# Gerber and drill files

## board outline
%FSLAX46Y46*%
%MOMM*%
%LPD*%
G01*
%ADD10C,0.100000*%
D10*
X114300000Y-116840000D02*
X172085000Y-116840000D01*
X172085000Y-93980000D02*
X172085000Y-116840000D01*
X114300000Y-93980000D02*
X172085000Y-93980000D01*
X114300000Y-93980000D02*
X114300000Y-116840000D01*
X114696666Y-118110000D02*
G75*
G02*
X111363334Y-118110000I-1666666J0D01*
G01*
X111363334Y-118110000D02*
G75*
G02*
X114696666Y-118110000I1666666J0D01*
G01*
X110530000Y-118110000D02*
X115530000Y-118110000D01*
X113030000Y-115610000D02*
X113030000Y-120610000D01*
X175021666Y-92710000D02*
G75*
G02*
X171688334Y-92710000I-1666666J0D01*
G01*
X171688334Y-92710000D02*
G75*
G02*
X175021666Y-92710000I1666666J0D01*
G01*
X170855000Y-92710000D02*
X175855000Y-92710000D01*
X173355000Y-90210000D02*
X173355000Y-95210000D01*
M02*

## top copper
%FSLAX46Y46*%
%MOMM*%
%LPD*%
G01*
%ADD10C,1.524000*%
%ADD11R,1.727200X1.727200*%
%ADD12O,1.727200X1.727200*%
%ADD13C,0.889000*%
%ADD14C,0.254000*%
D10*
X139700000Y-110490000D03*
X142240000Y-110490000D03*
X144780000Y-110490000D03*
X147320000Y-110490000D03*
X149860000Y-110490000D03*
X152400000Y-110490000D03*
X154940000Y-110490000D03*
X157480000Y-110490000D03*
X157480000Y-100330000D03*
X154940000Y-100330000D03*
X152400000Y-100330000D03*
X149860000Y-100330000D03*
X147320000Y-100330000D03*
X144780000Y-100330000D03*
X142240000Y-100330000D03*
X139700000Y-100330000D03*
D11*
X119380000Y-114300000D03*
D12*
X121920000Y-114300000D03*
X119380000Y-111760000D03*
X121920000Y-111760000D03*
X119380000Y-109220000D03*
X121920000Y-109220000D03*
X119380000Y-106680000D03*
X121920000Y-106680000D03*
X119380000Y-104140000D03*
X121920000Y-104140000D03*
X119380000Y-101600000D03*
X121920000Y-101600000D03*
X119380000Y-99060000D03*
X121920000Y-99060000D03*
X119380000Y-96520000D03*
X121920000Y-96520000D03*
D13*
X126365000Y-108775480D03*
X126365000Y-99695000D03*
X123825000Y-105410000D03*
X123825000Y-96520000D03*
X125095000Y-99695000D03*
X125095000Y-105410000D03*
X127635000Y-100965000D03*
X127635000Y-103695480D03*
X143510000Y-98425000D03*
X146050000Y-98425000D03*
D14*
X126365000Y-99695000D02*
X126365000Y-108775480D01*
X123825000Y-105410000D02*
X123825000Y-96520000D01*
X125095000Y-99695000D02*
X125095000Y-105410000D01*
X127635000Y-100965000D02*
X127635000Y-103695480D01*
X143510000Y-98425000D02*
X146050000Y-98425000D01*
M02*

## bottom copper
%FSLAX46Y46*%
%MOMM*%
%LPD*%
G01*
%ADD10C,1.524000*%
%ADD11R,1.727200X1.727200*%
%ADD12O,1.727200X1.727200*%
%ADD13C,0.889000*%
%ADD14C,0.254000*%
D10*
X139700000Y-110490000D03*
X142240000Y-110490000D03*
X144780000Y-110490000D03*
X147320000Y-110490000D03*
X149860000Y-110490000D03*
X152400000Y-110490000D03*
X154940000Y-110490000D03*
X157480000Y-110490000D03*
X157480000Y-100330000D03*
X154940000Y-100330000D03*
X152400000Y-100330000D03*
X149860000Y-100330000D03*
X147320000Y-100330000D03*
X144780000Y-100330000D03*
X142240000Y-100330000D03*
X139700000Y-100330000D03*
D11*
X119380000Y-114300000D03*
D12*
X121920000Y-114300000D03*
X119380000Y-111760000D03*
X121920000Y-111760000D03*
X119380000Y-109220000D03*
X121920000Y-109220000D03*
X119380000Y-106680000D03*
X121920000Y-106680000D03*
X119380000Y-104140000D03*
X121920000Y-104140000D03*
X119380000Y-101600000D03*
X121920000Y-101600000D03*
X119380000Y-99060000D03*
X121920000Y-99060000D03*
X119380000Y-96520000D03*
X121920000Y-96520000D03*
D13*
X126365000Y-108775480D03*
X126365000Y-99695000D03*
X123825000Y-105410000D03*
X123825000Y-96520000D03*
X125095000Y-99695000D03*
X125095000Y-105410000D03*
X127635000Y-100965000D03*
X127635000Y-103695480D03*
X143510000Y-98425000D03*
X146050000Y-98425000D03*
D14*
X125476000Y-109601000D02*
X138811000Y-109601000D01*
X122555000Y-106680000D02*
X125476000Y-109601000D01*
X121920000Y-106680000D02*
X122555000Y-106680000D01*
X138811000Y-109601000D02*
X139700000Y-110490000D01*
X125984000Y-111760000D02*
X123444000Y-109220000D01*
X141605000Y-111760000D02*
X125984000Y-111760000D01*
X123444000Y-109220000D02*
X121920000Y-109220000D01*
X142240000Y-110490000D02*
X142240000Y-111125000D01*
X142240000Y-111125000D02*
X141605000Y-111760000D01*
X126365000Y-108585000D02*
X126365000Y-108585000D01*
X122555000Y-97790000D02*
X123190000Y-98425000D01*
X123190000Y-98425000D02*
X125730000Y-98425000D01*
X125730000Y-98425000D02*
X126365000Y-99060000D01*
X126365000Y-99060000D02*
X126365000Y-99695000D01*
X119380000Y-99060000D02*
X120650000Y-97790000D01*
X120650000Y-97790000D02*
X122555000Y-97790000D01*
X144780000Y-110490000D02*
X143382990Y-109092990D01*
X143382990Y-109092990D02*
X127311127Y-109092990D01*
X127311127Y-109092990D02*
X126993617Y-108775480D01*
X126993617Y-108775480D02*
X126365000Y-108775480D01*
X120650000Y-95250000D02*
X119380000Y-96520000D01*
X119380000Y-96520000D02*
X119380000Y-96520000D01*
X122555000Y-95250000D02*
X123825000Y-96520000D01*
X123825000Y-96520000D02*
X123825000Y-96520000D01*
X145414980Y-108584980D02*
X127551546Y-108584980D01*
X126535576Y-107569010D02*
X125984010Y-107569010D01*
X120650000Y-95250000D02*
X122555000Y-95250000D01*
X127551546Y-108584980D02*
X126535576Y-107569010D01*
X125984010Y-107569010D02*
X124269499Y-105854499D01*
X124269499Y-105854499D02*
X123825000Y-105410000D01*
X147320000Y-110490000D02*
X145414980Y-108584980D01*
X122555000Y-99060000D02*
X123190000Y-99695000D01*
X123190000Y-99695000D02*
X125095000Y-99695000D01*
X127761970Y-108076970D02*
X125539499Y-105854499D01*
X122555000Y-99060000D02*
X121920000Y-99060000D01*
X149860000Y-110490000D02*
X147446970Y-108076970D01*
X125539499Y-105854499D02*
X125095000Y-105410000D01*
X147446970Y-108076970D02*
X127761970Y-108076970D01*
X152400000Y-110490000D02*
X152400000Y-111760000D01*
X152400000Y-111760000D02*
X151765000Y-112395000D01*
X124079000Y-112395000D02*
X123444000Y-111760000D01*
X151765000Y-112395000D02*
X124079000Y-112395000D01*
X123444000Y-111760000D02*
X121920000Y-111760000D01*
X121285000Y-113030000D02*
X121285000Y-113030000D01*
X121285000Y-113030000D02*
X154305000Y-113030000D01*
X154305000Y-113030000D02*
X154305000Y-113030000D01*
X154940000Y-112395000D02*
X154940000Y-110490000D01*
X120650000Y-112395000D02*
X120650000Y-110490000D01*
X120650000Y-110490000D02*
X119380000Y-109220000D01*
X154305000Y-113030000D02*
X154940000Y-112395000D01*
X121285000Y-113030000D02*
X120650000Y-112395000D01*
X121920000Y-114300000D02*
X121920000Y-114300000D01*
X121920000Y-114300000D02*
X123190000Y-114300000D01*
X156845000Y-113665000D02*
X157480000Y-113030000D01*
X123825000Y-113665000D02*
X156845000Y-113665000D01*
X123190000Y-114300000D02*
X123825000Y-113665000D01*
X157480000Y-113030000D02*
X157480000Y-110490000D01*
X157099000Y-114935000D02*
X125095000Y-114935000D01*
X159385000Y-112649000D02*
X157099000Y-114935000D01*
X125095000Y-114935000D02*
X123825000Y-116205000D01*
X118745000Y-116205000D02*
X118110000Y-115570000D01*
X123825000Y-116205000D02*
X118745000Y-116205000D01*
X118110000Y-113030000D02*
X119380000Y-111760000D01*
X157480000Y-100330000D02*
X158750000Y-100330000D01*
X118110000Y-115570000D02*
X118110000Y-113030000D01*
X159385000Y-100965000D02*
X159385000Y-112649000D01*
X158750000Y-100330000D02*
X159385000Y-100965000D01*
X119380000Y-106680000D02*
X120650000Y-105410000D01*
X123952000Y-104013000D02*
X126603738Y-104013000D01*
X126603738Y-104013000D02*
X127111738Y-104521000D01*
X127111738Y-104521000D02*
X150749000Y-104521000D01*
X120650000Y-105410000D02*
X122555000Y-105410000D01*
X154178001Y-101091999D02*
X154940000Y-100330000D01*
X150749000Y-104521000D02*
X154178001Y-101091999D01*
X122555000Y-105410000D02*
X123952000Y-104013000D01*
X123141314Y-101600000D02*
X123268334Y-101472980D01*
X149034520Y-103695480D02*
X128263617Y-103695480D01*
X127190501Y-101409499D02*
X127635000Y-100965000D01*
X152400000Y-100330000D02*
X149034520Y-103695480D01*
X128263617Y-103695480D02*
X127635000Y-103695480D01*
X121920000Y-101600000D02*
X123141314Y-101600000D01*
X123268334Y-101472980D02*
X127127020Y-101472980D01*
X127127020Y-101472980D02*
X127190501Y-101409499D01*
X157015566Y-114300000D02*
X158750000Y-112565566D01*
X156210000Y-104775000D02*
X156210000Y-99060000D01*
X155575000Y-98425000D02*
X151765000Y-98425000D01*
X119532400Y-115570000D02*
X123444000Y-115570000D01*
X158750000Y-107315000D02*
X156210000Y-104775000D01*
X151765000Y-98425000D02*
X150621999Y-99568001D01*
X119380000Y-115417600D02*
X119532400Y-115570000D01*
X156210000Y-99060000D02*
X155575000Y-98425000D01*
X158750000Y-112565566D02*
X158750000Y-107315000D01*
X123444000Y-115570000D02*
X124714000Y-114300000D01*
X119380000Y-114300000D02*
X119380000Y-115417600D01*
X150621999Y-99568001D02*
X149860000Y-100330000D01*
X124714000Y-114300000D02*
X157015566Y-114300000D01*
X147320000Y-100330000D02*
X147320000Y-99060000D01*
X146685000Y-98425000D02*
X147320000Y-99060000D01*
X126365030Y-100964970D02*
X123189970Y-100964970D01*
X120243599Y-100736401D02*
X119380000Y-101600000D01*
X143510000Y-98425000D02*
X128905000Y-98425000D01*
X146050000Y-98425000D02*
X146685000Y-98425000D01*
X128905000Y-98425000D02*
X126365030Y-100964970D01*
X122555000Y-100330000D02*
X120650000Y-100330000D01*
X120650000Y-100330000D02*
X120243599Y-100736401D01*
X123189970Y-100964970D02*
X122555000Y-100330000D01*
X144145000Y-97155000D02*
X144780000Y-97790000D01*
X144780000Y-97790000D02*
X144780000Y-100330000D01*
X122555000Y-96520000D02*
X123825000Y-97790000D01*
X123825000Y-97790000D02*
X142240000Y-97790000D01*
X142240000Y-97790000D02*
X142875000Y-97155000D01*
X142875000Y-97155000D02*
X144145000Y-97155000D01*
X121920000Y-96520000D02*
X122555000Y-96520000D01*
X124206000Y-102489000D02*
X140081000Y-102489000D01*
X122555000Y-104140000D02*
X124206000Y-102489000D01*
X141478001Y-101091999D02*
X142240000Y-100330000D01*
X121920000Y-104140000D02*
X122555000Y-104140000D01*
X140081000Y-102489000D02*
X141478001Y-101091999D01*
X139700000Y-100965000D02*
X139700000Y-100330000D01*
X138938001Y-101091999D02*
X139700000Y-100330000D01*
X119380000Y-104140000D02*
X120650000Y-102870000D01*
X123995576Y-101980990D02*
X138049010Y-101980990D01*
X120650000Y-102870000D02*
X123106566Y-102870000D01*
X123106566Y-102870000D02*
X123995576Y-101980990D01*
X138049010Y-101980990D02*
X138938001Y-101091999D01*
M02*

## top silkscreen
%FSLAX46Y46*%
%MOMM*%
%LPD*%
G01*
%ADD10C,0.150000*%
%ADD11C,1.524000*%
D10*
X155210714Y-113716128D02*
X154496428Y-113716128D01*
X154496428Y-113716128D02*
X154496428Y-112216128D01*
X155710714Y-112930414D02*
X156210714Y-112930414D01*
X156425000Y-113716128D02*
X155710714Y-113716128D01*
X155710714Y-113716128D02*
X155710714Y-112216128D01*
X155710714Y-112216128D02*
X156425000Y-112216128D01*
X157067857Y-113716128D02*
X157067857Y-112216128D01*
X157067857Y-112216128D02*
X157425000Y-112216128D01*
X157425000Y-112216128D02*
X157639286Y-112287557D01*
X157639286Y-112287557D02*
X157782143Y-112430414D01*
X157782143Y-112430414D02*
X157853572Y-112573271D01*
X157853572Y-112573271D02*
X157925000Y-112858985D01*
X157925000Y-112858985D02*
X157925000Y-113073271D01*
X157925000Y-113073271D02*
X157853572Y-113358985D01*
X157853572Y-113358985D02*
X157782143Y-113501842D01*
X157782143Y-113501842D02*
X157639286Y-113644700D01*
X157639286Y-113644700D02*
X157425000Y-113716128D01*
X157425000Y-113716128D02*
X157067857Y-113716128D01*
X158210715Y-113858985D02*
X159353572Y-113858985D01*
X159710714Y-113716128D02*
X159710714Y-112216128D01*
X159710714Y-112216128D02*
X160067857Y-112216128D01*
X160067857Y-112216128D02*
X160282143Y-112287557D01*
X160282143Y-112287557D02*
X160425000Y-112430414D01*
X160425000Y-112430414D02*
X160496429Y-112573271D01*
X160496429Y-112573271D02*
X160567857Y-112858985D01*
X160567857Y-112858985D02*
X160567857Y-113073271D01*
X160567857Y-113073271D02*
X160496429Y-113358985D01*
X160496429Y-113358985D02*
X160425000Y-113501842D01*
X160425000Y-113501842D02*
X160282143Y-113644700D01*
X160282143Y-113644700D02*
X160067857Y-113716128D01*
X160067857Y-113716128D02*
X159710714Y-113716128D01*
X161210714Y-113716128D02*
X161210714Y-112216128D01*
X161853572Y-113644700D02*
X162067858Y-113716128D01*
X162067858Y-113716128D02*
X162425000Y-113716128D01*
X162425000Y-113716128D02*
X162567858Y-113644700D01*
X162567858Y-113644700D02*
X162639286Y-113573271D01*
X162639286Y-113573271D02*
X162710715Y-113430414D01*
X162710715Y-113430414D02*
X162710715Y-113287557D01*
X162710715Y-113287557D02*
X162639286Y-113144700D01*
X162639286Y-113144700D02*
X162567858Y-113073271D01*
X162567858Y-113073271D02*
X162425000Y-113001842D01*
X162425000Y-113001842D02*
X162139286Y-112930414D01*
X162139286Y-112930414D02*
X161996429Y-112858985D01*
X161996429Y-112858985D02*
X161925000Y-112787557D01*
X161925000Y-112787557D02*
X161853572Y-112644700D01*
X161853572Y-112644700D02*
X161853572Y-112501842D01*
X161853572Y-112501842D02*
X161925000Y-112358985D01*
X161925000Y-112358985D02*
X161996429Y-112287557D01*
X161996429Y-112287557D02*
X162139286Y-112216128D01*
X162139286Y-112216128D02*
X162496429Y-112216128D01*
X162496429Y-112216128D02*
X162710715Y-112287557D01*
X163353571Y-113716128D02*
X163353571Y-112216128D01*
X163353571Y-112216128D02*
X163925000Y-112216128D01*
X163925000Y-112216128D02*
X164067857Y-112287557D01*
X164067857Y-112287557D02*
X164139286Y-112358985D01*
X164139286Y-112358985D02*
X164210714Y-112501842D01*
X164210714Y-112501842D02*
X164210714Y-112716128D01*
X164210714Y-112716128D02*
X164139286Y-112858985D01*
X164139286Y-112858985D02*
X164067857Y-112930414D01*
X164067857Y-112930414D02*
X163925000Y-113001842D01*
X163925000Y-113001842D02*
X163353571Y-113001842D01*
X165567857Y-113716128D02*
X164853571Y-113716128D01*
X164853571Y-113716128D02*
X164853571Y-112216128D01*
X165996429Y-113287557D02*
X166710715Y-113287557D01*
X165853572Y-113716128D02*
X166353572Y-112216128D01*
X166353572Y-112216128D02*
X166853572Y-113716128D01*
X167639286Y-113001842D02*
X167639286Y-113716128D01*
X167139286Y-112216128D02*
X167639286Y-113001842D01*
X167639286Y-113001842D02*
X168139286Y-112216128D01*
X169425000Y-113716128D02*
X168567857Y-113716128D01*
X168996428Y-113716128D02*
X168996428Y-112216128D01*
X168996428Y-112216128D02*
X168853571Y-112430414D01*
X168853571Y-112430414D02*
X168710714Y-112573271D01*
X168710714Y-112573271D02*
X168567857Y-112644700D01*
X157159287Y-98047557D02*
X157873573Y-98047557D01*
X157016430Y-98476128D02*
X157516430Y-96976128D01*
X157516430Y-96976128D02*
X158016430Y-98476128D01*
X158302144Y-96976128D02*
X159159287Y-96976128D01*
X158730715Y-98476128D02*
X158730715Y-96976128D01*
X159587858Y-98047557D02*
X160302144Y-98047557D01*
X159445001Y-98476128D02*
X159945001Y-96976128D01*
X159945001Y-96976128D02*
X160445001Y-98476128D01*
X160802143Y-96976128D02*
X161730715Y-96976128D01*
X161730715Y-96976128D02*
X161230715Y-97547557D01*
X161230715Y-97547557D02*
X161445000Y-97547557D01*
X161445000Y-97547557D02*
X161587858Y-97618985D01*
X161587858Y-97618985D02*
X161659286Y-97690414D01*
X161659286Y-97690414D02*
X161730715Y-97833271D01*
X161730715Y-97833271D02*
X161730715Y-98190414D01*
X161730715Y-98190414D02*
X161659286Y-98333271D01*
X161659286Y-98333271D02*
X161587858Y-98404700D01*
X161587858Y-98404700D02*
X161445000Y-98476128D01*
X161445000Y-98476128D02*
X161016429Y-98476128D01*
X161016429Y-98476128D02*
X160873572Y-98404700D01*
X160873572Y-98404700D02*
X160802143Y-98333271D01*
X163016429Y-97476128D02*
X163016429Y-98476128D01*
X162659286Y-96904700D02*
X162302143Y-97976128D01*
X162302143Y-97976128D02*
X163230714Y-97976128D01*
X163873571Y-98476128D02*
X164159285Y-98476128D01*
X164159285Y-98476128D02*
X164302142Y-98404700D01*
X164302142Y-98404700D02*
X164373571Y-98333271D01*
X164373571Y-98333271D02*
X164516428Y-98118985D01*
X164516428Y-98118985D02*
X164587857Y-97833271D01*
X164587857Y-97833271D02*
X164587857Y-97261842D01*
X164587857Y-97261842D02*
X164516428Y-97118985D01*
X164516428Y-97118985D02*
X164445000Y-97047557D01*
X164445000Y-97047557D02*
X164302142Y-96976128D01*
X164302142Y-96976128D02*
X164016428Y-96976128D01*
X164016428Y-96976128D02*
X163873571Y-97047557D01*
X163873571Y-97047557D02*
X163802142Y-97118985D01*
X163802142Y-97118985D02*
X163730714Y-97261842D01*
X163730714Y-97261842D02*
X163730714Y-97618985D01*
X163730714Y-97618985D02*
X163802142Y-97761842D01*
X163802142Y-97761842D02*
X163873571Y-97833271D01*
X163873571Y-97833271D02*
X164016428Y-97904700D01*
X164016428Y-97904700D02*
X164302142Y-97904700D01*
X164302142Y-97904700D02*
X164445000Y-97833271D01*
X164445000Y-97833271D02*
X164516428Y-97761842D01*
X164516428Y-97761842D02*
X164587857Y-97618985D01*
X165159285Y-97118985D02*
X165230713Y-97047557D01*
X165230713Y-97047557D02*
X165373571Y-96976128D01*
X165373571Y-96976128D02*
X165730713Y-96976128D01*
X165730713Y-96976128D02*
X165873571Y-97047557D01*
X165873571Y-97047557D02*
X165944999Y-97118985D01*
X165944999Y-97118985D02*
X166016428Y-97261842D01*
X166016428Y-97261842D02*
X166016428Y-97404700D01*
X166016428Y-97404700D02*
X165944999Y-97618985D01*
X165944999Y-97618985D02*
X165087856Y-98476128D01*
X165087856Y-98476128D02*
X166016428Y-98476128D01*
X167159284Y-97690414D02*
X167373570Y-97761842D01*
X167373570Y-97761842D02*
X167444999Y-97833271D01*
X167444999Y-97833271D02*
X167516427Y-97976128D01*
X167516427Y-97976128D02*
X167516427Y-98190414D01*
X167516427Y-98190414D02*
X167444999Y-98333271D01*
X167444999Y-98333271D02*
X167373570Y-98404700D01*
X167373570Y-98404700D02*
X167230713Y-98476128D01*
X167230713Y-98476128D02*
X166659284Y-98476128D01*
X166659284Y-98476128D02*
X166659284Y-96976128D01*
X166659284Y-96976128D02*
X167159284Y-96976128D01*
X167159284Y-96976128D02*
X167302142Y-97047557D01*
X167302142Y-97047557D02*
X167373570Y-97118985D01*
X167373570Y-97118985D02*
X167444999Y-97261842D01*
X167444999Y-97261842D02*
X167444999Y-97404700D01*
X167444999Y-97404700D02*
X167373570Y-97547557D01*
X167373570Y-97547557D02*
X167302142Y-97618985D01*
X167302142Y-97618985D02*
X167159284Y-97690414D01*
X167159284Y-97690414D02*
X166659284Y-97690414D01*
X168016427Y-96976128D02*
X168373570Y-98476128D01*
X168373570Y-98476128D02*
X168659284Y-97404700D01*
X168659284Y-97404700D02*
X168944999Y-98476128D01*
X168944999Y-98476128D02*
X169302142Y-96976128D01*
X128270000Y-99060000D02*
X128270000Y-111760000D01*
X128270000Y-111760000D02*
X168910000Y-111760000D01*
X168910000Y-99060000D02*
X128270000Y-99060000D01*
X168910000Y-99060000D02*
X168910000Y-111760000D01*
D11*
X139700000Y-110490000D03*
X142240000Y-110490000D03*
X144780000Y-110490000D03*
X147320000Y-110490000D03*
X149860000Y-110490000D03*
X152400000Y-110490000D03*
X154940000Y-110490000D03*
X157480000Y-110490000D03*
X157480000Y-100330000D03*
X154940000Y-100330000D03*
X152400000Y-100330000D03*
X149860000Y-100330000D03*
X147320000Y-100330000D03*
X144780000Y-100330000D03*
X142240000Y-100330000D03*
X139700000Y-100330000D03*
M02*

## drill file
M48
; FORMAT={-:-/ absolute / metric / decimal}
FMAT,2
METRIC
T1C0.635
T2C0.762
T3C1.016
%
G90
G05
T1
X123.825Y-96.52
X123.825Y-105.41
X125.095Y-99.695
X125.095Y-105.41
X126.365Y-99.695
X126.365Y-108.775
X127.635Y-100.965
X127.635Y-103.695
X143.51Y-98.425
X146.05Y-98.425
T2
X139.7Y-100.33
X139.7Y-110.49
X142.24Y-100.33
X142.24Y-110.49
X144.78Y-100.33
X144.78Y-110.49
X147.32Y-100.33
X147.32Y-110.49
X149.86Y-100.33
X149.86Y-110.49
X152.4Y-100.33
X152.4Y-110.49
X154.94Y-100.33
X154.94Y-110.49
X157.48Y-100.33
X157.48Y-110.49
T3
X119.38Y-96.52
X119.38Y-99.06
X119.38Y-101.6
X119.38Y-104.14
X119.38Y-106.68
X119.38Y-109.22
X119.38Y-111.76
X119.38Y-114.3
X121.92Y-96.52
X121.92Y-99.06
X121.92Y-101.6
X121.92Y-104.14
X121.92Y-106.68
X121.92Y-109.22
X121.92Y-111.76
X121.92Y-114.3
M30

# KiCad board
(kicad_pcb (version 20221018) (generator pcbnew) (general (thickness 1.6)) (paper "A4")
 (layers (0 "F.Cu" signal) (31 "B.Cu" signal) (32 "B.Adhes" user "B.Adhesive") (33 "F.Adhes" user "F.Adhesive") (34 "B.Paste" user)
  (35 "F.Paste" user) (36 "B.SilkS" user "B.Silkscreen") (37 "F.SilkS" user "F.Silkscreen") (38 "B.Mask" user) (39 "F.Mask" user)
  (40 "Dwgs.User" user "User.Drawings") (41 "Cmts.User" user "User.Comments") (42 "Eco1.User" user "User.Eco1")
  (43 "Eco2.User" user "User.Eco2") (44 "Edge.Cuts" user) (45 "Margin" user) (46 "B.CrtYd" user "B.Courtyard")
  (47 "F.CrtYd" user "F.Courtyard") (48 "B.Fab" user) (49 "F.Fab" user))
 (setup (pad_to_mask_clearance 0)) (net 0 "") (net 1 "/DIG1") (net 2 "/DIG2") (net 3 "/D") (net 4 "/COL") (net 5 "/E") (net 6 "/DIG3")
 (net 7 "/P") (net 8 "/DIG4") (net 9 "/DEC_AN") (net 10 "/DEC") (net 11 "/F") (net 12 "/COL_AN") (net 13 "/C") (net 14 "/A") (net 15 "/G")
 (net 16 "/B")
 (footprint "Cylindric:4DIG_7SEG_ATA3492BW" (layer "F.Cu") (at 148.59 105.41)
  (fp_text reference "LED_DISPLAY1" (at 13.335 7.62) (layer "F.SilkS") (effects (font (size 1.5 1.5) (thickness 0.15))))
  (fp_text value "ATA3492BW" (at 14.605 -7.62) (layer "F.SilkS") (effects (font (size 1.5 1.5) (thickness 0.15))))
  (fp_line (start -20.32 -6.35) (end -20.32 6.35) (stroke (width 0.15) (type solid)) (layer "F.SilkS"))
  (fp_line (start -20.32 6.35) (end 20.32 6.35) (stroke (width 0.15) (type solid)) (layer "F.SilkS"))
  (fp_line (start 20.32 -6.35) (end -20.32 -6.35) (stroke (width 0.15) (type solid)) (layer "F.SilkS"))
  (fp_line (start 20.32 -6.35) (end 20.32 6.35) (stroke (width 0.15) (type solid)) (layer "F.SilkS"))
  (pad "1" thru_hole circle (at -8.89 5.08) (size 1.524 1.524) (drill 0.762) (layers "*.Cu" "*.Mask" "F.SilkS") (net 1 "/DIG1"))
  (pad "2" thru_hole circle (at -6.35 5.08) (size 1.524 1.524) (drill 0.762) (layers "*.Cu" "*.Mask" "F.SilkS") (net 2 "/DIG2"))
  (pad "3" thru_hole circle (at -3.81 5.08) (size 1.524 1.524) (drill 0.762) (layers "*.Cu" "*.Mask" "F.SilkS") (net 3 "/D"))
  (pad "4" thru_hole circle (at -1.27 5.08) (size 1.524 1.524) (drill 0.762) (layers "*.Cu" "*.Mask" "F.SilkS") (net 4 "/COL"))
  (pad "5" thru_hole circle (at 1.27 5.08) (size 1.524 1.524) (drill 0.762) (layers "*.Cu" "*.Mask" "F.SilkS") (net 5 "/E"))
  (pad "6" thru_hole circle (at 3.81 5.08) (size 1.524 1.524) (drill 0.762) (layers "*.Cu" "*.Mask" "F.SilkS") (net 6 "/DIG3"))
  (pad "7" thru_hole circle (at 6.35 5.08) (size 1.524 1.524) (drill 0.762) (layers "*.Cu" "*.Mask" "F.SilkS") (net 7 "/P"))
  (pad "8" thru_hole circle (at 8.89 5.08) (size 1.524 1.524) (drill 0.762) (layers "*.Cu" "*.Mask" "F.SilkS") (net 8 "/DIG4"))
  (pad "9" thru_hole circle (at 8.89 -5.08) (size 1.524 1.524) (drill 0.762) (layers "*.Cu" "*.Mask" "F.SilkS") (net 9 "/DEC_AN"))
  (pad "10" thru_hole circle (at 6.35 -5.08) (size 1.524 1.524) (drill 0.762) (layers "*.Cu" "*.Mask" "F.SilkS") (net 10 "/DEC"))
  (pad "11" thru_hole circle (at 3.81 -5.08) (size 1.524 1.524) (drill 0.762) (layers "*.Cu" "*.Mask" "F.SilkS") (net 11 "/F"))
  (pad "12" thru_hole circle (at 1.27 -5.08) (size 1.524 1.524) (drill 0.762) (layers "*.Cu" "*.Mask" "F.SilkS") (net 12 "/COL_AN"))
  (pad "13" thru_hole circle (at -1.27 -5.08) (size 1.524 1.524) (drill 0.762) (layers "*.Cu" "*.Mask" "F.SilkS") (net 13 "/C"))
  (pad "14" thru_hole circle (at -3.81 -5.08) (size 1.524 1.524) (drill 0.762) (layers "*.Cu" "*.Mask" "F.SilkS") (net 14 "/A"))
  (pad "15" thru_hole circle (at -6.35 -5.08) (size 1.524 1.524) (drill 0.762) (layers "*.Cu" "*.Mask" "F.SilkS") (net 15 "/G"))
  (pad "16" thru_hole circle (at -8.89 -5.08) (size 1.524 1.524) (drill 0.762) (layers "*.Cu" "*.Mask" "F.SilkS") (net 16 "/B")))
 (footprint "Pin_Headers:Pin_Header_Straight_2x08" (layer "B.Cu") (at 120.65 105.41 90)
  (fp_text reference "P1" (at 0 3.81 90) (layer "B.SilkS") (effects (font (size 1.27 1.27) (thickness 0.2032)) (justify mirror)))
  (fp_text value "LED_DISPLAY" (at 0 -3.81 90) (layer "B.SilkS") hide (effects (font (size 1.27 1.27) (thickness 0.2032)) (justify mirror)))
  (pad "1" thru_hole rect (at -8.89 -1.27 90) (size 1.7272 1.7272) (drill 1.016) (layers "*.Cu" "*.Mask" "B.SilkS") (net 12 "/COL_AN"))
  (pad "2" thru_hole oval (at -8.89 1.27 90) (size 1.7272 1.7272) (drill 1.016) (layers "*.Cu" "*.Mask" "B.SilkS") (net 8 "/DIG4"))
  (pad "3" thru_hole oval (at -6.35 -1.27 90) (size 1.7272 1.7272) (drill 1.016) (layers "*.Cu" "*.Mask" "B.SilkS") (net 9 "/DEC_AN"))
  (pad "4" thru_hole oval (at -6.35 1.27 90) (size 1.7272 1.7272) (drill 1.016) (layers "*.Cu" "*.Mask" "B.SilkS") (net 6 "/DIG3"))
  (pad "5" thru_hole oval (at -3.81 -1.27 90) (size 1.7272 1.7272) (drill 1.016) (layers "*.Cu" "*.Mask" "B.SilkS") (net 7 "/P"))
  (pad "6" thru_hole oval (at -3.81 1.27 90) (size 1.7272 1.7272) (drill 1.016) (layers "*.Cu" "*.Mask" "B.SilkS") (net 2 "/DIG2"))
  (pad "7" thru_hole oval (at -1.27 -1.27 90) (size 1.7272 1.7272) (drill 1.016) (layers "*.Cu" "*.Mask" "B.SilkS") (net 10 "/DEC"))
  (pad "8" thru_hole oval (at -1.27 1.27 90) (size 1.7272 1.7272) (drill 1.016) (layers "*.Cu" "*.Mask" "B.SilkS") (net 1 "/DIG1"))
  (pad "9" thru_hole oval (at 1.27 -1.27 90) (size 1.7272 1.7272) (drill 1.016) (layers "*.Cu" "*.Mask" "B.SilkS") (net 16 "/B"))
  (pad "10" thru_hole oval (at 1.27 1.27 90) (size 1.7272 1.7272) (drill 1.016) (layers "*.Cu" "*.Mask" "B.SilkS") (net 15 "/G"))
  (pad "11" thru_hole oval (at 3.81 -1.27 90) (size 1.7272 1.7272) (drill 1.016) (layers "*.Cu" "*.Mask" "B.SilkS") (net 13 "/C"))
  (pad "12" thru_hole oval (at 3.81 1.27 90) (size 1.7272 1.7272) (drill 1.016) (layers "*.Cu" "*.Mask" "B.SilkS") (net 11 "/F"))
  (pad "13" thru_hole oval (at 6.35 -1.27 90) (size 1.7272 1.7272) (drill 1.016) (layers "*.Cu" "*.Mask" "B.SilkS") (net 3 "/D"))
  (pad "14" thru_hole oval (at 6.35 1.27 90) (size 1.7272 1.7272) (drill 1.016) (layers "*.Cu" "*.Mask" "B.SilkS") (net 5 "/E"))
  (pad "15" thru_hole oval (at 8.89 -1.27 90) (size 1.7272 1.7272) (drill 1.016) (layers "*.Cu" "*.Mask" "B.SilkS") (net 4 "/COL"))
  (pad "16" thru_hole oval (at 8.89 1.27 90) (size 1.7272 1.7272) (drill 1.016) (layers "*.Cu" "*.Mask" "B.SilkS") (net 14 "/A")))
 (gr_line (start 114.3 116.84) (end 172.085 116.84) (stroke (width 0.1) (type solid)) (layer "Edge.Cuts"))
 (gr_line (start 172.085 93.98) (end 172.085 116.84) (stroke (width 0.1) (type solid)) (layer "Edge.Cuts"))
 (gr_line (start 114.3 93.98) (end 172.085 93.98) (stroke (width 0.1) (type solid)) (layer "Edge.Cuts"))
 (gr_line (start 114.3 93.98) (end 114.3 116.84) (stroke (width 0.1) (type solid)) (layer "Edge.Cuts"))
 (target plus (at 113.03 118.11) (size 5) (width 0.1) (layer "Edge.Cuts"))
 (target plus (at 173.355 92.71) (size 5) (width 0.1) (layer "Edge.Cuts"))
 (segment (start 125.476 109.601) (end 138.811 109.601) (width 0.254) (layer "B.Cu") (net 1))
 (segment (start 122.555 106.68) (end 125.476 109.601) (width 0.254) (layer "B.Cu") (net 1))
 (segment (start 121.92 106.68) (end 122.555 106.68) (width 0.254) (layer "B.Cu") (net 1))
 (segment (start 138.811 109.601) (end 139.7 110.49) (width 0.254) (layer "B.Cu") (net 1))
 (segment (start 125.984 111.76) (end 123.444 109.22) (width 0.254) (layer "B.Cu") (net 2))
 (segment (start 141.605 111.76) (end 125.984 111.76) (width 0.254) (layer "B.Cu") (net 2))
 (segment (start 123.444 109.22) (end 121.92 109.22) (width 0.254) (layer "B.Cu") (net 2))
 (segment (start 142.24 110.49) (end 142.24 111.125) (width 0.254) (layer "B.Cu") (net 2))
 (segment (start 142.24 111.125) (end 141.605 111.76) (width 0.254) (layer "B.Cu") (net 2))
 (segment (start 126.365 99.695) (end 126.365 108.77548) (width 0.254) (layer "F.Cu") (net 3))
 (via (at 126.365 108.77548) (size 0.889) (drill 0.635) (layers "F.Cu" "B.Cu") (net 3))
 (via (at 126.365 99.695) (size 0.889) (drill 0.635) (layers "F.Cu" "B.Cu") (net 3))
 (segment (start 126.365 108.585) (end 126.365 108.585) (width 0.254) (layer "B.Cu") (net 3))
 (segment (start 122.555 97.79) (end 123.19 98.425) (width 0.254) (layer "B.Cu") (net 3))
 (segment (start 123.19 98.425) (end 125.73 98.425) (width 0.254) (layer "B.Cu") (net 3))
 (segment (start 125.73 98.425) (end 126.365 99.06) (width 0.254) (layer "B.Cu") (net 3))
 (segment (start 126.365 99.06) (end 126.365 99.695) (width 0.254) (layer "B.Cu") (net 3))
 (segment (start 119.38 99.06) (end 120.65 97.79) (width 0.254) (layer "B.Cu") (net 3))
 (segment (start 120.65 97.79) (end 122.555 97.79) (width 0.254) (layer "B.Cu") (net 3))
 (segment (start 144.78 110.49) (end 143.38299 109.09299) (width 0.254) (layer "B.Cu") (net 3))
 (segment (start 143.38299 109.09299) (end 127.311127 109.09299) (width 0.254) (layer "B.Cu") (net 3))
 (segment (start 127.311127 109.09299) (end 126.993617 108.77548) (width 0.254) (layer "B.Cu") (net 3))
 (segment (start 126.993617 108.77548) (end 126.365 108.77548) (width 0.254) (layer "B.Cu") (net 3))
 (segment (start 123.825 105.41) (end 123.825 96.52) (width 0.254) (layer "F.Cu") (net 4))
 (via (at 123.825 105.41) (size 0.889) (drill 0.635) (layers "F.Cu" "B.Cu") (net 4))
 (via (at 123.825 96.52) (size 0.889) (drill 0.635) (layers "F.Cu" "B.Cu") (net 4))
 (segment (start 120.65 95.25) (end 119.38 96.52) (width 0.254) (layer "B.Cu") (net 4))
 (segment (start 119.38 96.52) (end 119.38 96.52) (width 0.254) (layer "B.Cu") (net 4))
 (segment (start 122.555 95.25) (end 123.825 96.52) (width 0.254) (layer "B.Cu") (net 4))
 (segment (start 123.825 96.52) (end 123.825 96.52) (width 0.254) (layer "B.Cu") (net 4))
 (segment (start 145.41498 108.58498) (end 127.551546 108.58498) (width 0.254) (layer "B.Cu") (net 4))
 (segment (start 126.535576 107.56901) (end 125.98401 107.56901) (width 0.254) (layer "B.Cu") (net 4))
 (segment (start 120.65 95.25) (end 122.555 95.25) (width 0.254) (layer "B.Cu") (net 4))
 (segment (start 127.551546 108.58498) (end 126.535576 107.56901) (width 0.254) (layer "B.Cu") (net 4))
 (segment (start 125.98401 107.56901) (end 124.269499 105.854499) (width 0.254) (layer "B.Cu") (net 4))
 (segment (start 124.269499 105.854499) (end 123.825 105.41) (width 0.254) (layer "B.Cu") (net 4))
 (segment (start 147.32 110.49) (end 145.41498 108.58498) (width 0.254) (layer "B.Cu") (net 4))
 (segment (start 125.095 99.695) (end 125.095 105.41) (width 0.254) (layer "F.Cu") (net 5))
 (via (at 125.095 99.695) (size 0.889) (drill 0.635) (layers "F.Cu" "B.Cu") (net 5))
 (via (at 125.095 105.41) (size 0.889) (drill 0.635) (layers "F.Cu" "B.Cu") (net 5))
 (segment (start 122.555 99.06) (end 123.19 99.695) (width 0.254) (layer "B.Cu") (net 5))
 (segment (start 123.19 99.695) (end 125.095 99.695) (width 0.254) (layer "B.Cu") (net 5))
 (segment (start 127.76197 108.07697) (end 125.539499 105.854499) (width 0.254) (layer "B.Cu") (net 5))
 (segment (start 122.555 99.06) (end 121.92 99.06) (width 0.254) (layer "B.Cu") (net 5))
 (segment (start 149.86 110.49) (end 147.44697 108.07697) (width 0.254) (layer "B.Cu") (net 5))
 (segment (start 125.539499 105.854499) (end 125.095 105.41) (width 0.254) (layer "B.Cu") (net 5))
 (segment (start 147.44697 108.07697) (end 127.76197 108.07697) (width 0.254) (layer "B.Cu") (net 5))
 (segment (start 152.4 110.49) (end 152.4 111.76) (width 0.254) (layer "B.Cu") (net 6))
 (segment (start 152.4 111.76) (end 151.765 112.395) (width 0.254) (layer "B.Cu") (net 6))
 (segment (start 124.079 112.395) (end 123.444 111.76) (width 0.254) (layer "B.Cu") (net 6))
 (segment (start 151.765 112.395) (end 124.079 112.395) (width 0.254) (layer "B.Cu") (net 6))
 (segment (start 123.444 111.76) (end 121.92 111.76) (width 0.254) (layer "B.Cu") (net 6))
 (segment (start 121.285 113.03) (end 121.285 113.03) (width 0.254) (layer "B.Cu") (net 7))
 (segment (start 121.285 113.03) (end 154.305 113.03) (width 0.254) (layer "B.Cu") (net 7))
 (segment (start 154.305 113.03) (end 154.305 113.03) (width 0.254) (layer "B.Cu") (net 7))
 (segment (start 154.94 112.395) (end 154.94 110.49) (width 0.254) (layer "B.Cu") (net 7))
 (segment (start 120.65 112.395) (end 120.65 110.49) (width 0.254) (layer "B.Cu") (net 7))
 (segment (start 120.65 110.49) (end 119.38 109.22) (width 0.254) (layer "B.Cu") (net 7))
 (segment (start 154.305 113.03) (end 154.94 112.395) (width 0.254) (layer "B.Cu") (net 7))
 (segment (start 121.285 113.03) (end 120.65 112.395) (width 0.254) (layer "B.Cu") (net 7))
 (segment (start 121.92 114.3) (end 121.92 114.3) (width 0.254) (layer "B.Cu") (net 8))
 (segment (start 121.92 114.3) (end 123.19 114.3) (width 0.254) (layer "B.Cu") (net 8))
 (segment (start 156.845 113.665) (end 157.48 113.03) (width 0.254) (layer "B.Cu") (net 8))
 (segment (start 123.825 113.665) (end 156.845 113.665) (width 0.254) (layer "B.Cu") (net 8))
 (segment (start 123.19 114.3) (end 123.825 113.665) (width 0.254) (layer "B.Cu") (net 8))
 (segment (start 157.48 113.03) (end 157.48 110.49) (width 0.254) (layer "B.Cu") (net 8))
 (segment (start 157.099 114.935) (end 125.095 114.935) (width 0.254) (layer "B.Cu") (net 9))
 (segment (start 159.385 112.649) (end 157.099 114.935) (width 0.254) (layer "B.Cu") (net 9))
 (segment (start 125.095 114.935) (end 123.825 116.205) (width 0.254) (layer "B.Cu") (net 9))
 (segment (start 118.745 116.205) (end 118.11 115.57) (width 0.254) (layer "B.Cu") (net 9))
 (segment (start 123.825 116.205) (end 118.745 116.205) (width 0.254) (layer "B.Cu") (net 9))
 (segment (start 118.11 113.03) (end 119.38 111.76) (width 0.254) (layer "B.Cu") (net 9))
 (segment (start 157.48 100.33) (end 158.75 100.33) (width 0.254) (layer "B.Cu") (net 9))
 (segment (start 118.11 115.57) (end 118.11 113.03) (width 0.254) (layer "B.Cu") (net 9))
 (segment (start 159.385 100.965) (end 159.385 112.649) (width 0.254) (layer "B.Cu") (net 9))
 (segment (start 158.75 100.33) (end 159.385 100.965) (width 0.254) (layer "B.Cu") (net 9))
 (segment (start 119.38 106.68) (end 120.65 105.41) (width 0.254) (layer "B.Cu") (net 10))
 (segment (start 123.952 104.013) (end 126.603738 104.013) (width 0.254) (layer "B.Cu") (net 10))
 (segment (start 126.603738 104.013) (end 127.111738 104.521) (width 0.254) (layer "B.Cu") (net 10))
 (segment (start 127.111738 104.521) (end 150.749 104.521) (width 0.254) (layer "B.Cu") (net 10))
 (segment (start 120.65 105.41) (end 122.555 105.41) (width 0.254) (layer "B.Cu") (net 10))
 (segment (start 154.178001 101.091999) (end 154.94 100.33) (width 0.254) (layer "B.Cu") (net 10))
 (segment (start 150.749 104.521) (end 154.178001 101.091999) (width 0.254) (layer "B.Cu") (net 10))
 (segment (start 122.555 105.41) (end 123.952 104.013) (width 0.254) (layer "B.Cu") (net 10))
 (segment (start 127.635 100.965) (end 127.635 103.69548) (width 0.254) (layer "F.Cu") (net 11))
 (via (at 127.635 100.965) (size 0.889) (drill 0.635) (layers "F.Cu" "B.Cu") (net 11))
 (via (at 127.635 103.69548) (size 0.889) (drill 0.635) (layers "F.Cu" "B.Cu") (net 11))
 (segment (start 123.141314 101.6) (end 123.268334 101.47298) (width 0.254) (layer "B.Cu") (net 11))
 (segment (start 149.03452 103.69548) (end 128.263617 103.69548) (width 0.254) (layer "B.Cu") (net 11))
 (segment (start 127.190501 101.409499) (end 127.635 100.965) (width 0.254) (layer "B.Cu") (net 11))
 (segment (start 152.4 100.33) (end 149.03452 103.69548) (width 0.254) (layer "B.Cu") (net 11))
 (segment (start 128.263617 103.69548) (end 127.635 103.69548) (width 0.254) (layer "B.Cu") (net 11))
 (segment (start 121.92 101.6) (end 123.141314 101.6) (width 0.254) (layer "B.Cu") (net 11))
 (segment (start 123.268334 101.47298) (end 127.12702 101.47298) (width 0.254) (layer "B.Cu") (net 11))
 (segment (start 127.12702 101.47298) (end 127.190501 101.409499) (width 0.254) (layer "B.Cu") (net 11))
 (segment (start 157.015566 114.3) (end 158.75 112.565566) (width 0.254) (layer "B.Cu") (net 12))
 (segment (start 156.21 104.775) (end 156.21 99.06) (width 0.254) (layer "B.Cu") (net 12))
 (segment (start 155.575 98.425) (end 151.765 98.425) (width 0.254) (layer "B.Cu") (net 12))
 (segment (start 119.5324 115.57) (end 123.444 115.57) (width 0.254) (layer "B.Cu") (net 12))
 (segment (start 158.75 107.315) (end 156.21 104.775) (width 0.254) (layer "B.Cu") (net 12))
 (segment (start 151.765 98.425) (end 150.621999 99.568001) (width 0.254) (layer "B.Cu") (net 12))
 (segment (start 119.38 115.4176) (end 119.5324 115.57) (width 0.254) (layer "B.Cu") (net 12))
 (segment (start 156.21 99.06) (end 155.575 98.425) (width 0.254) (layer "B.Cu") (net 12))
 (segment (start 158.75 112.565566) (end 158.75 107.315) (width 0.254) (layer "B.Cu") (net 12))
 (segment (start 123.444 115.57) (end 124.714 114.3) (width 0.254) (layer "B.Cu") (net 12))
 (segment (start 119.38 114.3) (end 119.38 115.4176) (width 0.254) (layer "B.Cu") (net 12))
 (segment (start 150.621999 99.568001) (end 149.86 100.33) (width 0.254) (layer "B.Cu") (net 12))
 (segment (start 124.714 114.3) (end 157.015566 114.3) (width 0.254) (layer "B.Cu") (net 12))
 (segment (start 143.51 98.425) (end 146.05 98.425) (width 0.254) (layer "F.Cu") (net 13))
 (via (at 143.51 98.425) (size 0.889) (drill 0.635) (layers "F.Cu" "B.Cu") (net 13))
 (via (at 146.05 98.425) (size 0.889) (drill 0.635) (layers "F.Cu" "B.Cu") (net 13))
 (segment (start 147.32 100.33) (end 147.32 99.06) (width 0.254) (layer "B.Cu") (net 13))
 (segment (start 146.685 98.425) (end 147.32 99.06) (width 0.254) (layer "B.Cu") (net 13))
 (segment (start 126.36503 100.96497) (end 123.18997 100.96497) (width 0.254) (layer "B.Cu") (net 13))
 (segment (start 120.243599 100.736401) (end 119.38 101.6) (width 0.254) (layer "B.Cu") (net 13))
 (segment (start 143.51 98.425) (end 128.905 98.425) (width 0.254) (layer "B.Cu") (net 13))
 (segment (start 146.05 98.425) (end 146.685 98.425) (width 0.254) (layer "B.Cu") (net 13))
 (segment (start 128.905 98.425) (end 126.36503 100.96497) (width 0.254) (layer "B.Cu") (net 13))
 (segment (start 122.555 100.33) (end 120.65 100.33) (width 0.254) (layer "B.Cu") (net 13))
 (segment (start 120.65 100.33) (end 120.243599 100.736401) (width 0.254) (layer "B.Cu") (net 13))
 (segment (start 123.18997 100.96497) (end 122.555 100.33) (width 0.254) (layer "B.Cu") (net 13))
 (segment (start 144.145 97.155) (end 144.78 97.79) (width 0.254) (layer "B.Cu") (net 14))
 (segment (start 144.78 97.79) (end 144.78 100.33) (width 0.254) (layer "B.Cu") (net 14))
 (segment (start 122.555 96.52) (end 123.825 97.79) (width 0.254) (layer "B.Cu") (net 14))
 (segment (start 123.825 97.79) (end 142.24 97.79) (width 0.254) (layer "B.Cu") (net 14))
 (segment (start 142.24 97.79) (end 142.875 97.155) (width 0.254) (layer "B.Cu") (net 14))
 (segment (start 142.875 97.155) (end 144.145 97.155) (width 0.254) (layer "B.Cu") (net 14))
 (segment (start 121.92 96.52) (end 122.555 96.52) (width 0.254) (layer "B.Cu") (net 14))
 (segment (start 124.206 102.489) (end 140.081 102.489) (width 0.254) (layer "B.Cu") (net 15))
 (segment (start 122.555 104.14) (end 124.206 102.489) (width 0.254) (layer "B.Cu") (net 15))
 (segment (start 141.478001 101.091999) (end 142.24 100.33) (width 0.254) (layer "B.Cu") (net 15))
 (segment (start 121.92 104.14) (end 122.555 104.14) (width 0.254) (layer "B.Cu") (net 15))
 (segment (start 140.081 102.489) (end 141.478001 101.091999) (width 0.254) (layer "B.Cu") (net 15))
 (segment (start 139.7 100.965) (end 139.7 100.33) (width 0.254) (layer "B.Cu") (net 16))
 (segment (start 138.938001 101.091999) (end 139.7 100.33) (width 0.254) (layer "B.Cu") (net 16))
 (segment (start 119.38 104.14) (end 120.65 102.87) (width 0.254) (layer "B.Cu") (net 16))
 (segment (start 123.995576 101.98099) (end 138.04901 101.98099) (width 0.254) (layer "B.Cu") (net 16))
 (segment (start 120.65 102.87) (end 123.106566 102.87) (width 0.254) (layer "B.Cu") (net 16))
 (segment (start 123.106566 102.87) (end 123.995576 101.98099) (width 0.254) (layer "B.Cu") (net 16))
 (segment (start 138.04901 101.98099) (end 138.938001 101.091999) (width 0.254) (layer "B.Cu") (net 16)))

